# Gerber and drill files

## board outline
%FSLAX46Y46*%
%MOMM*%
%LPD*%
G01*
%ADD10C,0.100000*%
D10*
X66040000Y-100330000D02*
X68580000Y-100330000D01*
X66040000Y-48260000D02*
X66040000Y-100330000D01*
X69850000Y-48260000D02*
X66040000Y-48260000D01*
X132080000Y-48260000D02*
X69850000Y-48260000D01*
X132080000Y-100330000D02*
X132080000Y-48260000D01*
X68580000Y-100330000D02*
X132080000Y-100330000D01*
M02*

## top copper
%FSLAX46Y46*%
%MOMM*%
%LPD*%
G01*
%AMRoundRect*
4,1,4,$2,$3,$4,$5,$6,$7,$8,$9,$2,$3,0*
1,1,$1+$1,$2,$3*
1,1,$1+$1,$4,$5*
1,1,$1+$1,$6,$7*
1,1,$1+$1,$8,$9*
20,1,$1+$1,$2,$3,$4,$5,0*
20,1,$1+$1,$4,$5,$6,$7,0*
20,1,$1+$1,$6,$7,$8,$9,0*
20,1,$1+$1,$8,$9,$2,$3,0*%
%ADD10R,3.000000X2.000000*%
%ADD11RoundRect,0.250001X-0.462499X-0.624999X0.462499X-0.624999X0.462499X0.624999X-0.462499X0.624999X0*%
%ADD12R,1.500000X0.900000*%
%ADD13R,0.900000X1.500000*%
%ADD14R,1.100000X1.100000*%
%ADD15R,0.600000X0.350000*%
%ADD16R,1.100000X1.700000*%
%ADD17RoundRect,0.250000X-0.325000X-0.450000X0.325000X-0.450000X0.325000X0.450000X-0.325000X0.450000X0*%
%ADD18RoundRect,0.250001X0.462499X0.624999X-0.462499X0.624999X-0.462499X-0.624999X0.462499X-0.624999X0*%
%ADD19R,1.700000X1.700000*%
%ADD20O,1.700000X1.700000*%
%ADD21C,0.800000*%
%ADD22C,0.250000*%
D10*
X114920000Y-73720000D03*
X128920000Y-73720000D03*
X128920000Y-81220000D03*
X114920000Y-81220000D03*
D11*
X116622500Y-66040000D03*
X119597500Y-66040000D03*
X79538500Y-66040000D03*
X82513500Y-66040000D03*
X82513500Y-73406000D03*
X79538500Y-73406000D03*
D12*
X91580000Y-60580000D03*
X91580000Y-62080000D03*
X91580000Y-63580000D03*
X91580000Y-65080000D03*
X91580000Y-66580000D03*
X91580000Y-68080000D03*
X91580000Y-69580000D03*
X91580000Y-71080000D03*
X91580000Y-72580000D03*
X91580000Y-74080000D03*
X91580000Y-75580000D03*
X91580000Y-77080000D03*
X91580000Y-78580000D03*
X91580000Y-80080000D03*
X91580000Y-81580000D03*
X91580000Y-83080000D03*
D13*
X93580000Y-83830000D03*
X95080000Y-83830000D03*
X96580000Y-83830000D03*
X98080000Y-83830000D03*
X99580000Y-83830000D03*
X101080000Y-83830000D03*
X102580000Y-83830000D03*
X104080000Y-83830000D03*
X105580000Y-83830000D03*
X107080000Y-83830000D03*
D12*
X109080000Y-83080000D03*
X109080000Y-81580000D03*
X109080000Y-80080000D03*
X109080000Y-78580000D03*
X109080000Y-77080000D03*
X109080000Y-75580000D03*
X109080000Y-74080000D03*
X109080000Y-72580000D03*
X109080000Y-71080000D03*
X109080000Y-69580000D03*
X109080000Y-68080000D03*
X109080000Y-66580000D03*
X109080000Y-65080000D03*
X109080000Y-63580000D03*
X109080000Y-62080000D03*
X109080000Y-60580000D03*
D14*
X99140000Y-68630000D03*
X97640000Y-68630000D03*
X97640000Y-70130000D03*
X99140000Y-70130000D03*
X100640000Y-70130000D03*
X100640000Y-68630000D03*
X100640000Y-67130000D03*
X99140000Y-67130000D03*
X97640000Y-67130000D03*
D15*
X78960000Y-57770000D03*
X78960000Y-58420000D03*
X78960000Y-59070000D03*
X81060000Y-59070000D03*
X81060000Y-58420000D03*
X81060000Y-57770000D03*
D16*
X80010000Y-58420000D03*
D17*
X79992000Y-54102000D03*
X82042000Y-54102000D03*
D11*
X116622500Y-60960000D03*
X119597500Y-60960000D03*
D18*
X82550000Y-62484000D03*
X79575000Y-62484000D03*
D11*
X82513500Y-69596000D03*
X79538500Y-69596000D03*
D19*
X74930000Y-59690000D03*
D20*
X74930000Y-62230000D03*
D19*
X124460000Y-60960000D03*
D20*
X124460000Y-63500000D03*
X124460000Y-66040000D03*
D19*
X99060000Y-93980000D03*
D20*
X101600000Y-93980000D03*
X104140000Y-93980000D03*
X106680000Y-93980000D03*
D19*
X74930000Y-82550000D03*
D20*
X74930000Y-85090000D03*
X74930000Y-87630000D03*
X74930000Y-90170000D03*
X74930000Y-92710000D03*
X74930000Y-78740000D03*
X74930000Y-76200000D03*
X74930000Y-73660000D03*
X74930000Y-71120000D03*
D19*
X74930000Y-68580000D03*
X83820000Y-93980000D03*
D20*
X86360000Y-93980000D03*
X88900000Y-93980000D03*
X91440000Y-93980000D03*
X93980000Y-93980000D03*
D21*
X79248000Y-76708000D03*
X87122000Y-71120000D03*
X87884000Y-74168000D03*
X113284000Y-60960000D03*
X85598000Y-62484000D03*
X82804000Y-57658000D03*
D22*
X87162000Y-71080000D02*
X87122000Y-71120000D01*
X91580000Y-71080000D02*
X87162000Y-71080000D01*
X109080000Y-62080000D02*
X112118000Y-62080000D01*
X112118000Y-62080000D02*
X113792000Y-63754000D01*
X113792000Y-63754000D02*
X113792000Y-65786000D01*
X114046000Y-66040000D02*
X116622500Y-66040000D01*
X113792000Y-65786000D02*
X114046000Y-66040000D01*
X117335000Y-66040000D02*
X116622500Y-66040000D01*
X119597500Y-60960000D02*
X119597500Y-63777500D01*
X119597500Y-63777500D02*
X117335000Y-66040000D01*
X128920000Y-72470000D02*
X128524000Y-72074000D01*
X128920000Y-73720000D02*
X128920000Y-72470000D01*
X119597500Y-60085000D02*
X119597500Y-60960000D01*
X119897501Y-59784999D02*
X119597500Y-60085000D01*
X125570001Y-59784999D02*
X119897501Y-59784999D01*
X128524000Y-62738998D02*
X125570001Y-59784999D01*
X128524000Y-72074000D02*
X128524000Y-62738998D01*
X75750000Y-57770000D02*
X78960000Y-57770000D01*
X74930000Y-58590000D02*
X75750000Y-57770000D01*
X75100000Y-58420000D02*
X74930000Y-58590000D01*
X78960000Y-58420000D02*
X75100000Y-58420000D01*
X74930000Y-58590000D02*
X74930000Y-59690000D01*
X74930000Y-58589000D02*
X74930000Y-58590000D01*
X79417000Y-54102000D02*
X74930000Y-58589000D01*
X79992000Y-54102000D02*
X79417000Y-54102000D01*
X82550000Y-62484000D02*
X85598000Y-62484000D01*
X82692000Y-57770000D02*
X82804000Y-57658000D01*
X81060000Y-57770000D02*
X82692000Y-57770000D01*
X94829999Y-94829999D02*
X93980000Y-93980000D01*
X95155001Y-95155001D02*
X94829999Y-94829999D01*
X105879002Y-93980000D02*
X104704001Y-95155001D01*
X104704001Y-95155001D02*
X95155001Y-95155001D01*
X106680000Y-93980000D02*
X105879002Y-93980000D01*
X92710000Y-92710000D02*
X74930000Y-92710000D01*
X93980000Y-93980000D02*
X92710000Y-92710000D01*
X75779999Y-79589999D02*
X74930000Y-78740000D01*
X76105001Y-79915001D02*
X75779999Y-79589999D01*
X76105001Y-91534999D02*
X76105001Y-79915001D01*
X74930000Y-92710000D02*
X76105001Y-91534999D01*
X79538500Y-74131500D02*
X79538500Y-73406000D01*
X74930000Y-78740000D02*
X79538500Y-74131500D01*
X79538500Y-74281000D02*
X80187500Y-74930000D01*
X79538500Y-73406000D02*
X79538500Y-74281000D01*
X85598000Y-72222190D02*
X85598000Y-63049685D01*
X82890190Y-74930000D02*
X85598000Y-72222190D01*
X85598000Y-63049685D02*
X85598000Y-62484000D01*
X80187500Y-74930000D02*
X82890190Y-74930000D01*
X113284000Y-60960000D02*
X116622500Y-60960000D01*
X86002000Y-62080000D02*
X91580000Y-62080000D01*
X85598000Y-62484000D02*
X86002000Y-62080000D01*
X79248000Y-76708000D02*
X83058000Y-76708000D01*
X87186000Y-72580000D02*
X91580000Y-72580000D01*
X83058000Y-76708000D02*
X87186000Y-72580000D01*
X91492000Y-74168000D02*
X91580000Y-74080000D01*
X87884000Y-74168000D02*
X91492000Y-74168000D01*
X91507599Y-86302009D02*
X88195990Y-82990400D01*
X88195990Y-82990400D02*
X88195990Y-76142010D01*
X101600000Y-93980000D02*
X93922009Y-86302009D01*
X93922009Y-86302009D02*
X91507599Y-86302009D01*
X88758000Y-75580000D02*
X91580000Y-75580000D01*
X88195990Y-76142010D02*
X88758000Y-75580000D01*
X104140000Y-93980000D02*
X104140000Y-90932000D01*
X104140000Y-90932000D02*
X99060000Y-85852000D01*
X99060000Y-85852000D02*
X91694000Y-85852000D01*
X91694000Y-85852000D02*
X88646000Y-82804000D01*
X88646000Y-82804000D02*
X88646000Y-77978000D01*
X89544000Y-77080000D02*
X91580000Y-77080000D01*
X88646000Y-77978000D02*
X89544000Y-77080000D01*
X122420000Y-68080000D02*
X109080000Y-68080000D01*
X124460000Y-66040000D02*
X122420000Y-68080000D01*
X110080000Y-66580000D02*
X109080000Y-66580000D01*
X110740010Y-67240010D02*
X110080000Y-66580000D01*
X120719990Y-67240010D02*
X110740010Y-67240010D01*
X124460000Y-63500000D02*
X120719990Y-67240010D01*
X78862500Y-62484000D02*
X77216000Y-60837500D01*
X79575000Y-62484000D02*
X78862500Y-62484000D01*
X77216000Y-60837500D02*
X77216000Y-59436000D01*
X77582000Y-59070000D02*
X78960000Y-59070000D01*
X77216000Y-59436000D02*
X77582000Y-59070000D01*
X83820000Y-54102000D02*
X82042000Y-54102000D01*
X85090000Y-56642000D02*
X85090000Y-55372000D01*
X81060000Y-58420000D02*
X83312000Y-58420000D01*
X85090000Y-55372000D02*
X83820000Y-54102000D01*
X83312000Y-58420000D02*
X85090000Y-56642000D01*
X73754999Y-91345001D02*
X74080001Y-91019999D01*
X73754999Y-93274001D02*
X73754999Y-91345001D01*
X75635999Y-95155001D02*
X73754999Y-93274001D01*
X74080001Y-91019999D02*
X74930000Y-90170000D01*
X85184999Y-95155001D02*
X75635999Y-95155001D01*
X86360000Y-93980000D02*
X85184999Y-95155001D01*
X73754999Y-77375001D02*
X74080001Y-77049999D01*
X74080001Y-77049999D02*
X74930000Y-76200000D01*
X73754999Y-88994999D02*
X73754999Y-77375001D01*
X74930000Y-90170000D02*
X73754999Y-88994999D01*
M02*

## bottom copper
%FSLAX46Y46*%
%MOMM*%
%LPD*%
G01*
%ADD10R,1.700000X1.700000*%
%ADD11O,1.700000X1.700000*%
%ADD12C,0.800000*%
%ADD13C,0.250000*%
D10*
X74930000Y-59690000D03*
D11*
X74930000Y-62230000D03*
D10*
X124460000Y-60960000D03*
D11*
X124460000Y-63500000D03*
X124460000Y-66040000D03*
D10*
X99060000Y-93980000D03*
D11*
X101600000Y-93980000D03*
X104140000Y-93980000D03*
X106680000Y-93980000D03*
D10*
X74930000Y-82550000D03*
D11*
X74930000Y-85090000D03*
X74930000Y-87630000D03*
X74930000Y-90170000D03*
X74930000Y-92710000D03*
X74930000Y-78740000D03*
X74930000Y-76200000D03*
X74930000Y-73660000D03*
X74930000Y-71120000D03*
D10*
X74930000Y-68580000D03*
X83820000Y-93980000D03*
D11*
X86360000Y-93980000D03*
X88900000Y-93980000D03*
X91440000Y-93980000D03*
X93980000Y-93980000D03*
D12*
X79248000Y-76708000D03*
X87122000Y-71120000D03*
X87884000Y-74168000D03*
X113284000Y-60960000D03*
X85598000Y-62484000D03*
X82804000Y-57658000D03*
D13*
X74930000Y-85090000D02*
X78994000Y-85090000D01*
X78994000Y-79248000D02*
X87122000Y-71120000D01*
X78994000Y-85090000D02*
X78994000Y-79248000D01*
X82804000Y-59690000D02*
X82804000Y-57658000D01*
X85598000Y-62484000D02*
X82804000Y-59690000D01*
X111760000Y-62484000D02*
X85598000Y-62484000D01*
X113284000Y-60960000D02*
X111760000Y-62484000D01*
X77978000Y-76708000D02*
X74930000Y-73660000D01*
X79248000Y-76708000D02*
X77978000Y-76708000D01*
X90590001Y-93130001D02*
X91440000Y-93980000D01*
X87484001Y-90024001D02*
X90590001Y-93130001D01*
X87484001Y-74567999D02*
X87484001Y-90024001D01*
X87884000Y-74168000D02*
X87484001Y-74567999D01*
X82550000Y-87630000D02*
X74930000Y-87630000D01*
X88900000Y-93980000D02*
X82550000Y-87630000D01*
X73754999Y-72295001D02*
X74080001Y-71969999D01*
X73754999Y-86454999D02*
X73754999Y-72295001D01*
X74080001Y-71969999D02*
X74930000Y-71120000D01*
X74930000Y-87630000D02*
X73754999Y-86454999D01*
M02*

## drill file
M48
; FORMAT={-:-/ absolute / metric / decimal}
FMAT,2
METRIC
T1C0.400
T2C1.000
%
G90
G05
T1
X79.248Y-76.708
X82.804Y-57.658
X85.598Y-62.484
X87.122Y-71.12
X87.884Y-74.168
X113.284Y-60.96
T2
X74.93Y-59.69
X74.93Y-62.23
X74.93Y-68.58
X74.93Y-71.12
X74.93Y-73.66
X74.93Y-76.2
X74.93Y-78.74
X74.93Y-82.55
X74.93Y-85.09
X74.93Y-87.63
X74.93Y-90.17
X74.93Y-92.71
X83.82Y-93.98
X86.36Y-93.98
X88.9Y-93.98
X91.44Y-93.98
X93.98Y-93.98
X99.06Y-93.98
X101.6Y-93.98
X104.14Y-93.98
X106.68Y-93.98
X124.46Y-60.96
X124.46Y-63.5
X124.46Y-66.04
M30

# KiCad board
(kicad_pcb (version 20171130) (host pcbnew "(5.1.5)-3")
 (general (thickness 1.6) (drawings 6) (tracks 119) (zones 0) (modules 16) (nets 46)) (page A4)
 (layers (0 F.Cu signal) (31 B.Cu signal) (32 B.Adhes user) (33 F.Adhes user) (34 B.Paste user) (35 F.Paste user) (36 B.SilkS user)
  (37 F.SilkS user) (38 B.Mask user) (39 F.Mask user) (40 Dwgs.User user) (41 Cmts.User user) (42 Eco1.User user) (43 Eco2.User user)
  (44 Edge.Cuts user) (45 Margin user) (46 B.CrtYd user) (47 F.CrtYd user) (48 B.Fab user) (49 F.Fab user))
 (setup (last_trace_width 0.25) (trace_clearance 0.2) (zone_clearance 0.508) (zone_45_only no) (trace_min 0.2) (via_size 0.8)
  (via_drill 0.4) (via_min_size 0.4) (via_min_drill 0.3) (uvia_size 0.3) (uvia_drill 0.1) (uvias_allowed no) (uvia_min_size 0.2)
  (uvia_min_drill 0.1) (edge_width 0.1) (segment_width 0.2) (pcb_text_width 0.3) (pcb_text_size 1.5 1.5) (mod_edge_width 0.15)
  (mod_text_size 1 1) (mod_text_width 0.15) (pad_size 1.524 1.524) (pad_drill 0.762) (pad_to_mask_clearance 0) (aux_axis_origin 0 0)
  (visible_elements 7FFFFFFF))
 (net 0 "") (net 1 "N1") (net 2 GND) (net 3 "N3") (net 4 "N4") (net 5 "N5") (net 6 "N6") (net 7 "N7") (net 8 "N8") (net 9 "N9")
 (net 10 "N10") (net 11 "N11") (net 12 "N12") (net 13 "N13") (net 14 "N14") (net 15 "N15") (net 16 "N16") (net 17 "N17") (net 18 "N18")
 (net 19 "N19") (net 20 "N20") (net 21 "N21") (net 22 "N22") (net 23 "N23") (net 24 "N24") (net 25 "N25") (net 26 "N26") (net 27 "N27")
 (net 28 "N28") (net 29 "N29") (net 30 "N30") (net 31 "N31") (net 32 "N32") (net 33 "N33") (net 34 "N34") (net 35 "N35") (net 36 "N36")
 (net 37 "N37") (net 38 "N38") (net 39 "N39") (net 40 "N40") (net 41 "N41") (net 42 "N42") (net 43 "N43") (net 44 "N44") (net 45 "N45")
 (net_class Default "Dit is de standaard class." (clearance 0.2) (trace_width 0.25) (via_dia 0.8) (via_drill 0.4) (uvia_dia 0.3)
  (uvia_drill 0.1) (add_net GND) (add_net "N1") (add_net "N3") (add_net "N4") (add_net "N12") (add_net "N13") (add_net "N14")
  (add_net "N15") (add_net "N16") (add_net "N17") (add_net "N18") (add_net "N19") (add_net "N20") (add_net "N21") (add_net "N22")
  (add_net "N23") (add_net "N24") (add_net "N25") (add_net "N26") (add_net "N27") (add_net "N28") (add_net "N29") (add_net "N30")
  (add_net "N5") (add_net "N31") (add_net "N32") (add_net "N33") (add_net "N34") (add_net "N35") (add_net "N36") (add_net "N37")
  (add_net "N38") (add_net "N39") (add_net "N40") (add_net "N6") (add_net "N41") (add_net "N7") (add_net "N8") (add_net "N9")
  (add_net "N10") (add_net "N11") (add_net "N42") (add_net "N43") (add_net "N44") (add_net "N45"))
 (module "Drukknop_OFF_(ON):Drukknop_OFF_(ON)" (layer F.Cu) (at 121.92 77.47)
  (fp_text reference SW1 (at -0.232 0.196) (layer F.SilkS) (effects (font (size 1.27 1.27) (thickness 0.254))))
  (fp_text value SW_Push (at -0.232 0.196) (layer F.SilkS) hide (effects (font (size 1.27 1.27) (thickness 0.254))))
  (pad 4 smd rect (at -7 -3.75 90) (size 2 3) (layers F.Cu F.Paste F.Mask))
  (pad 3 smd rect (at 7 -3.75 90) (size 2 3) (layers F.Cu F.Paste F.Mask) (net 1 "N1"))
  (pad 2 smd rect (at 7 3.75 90) (size 2 3) (layers F.Cu F.Paste F.Mask))
  (pad 1 smd rect (at -7 3.75 90) (size 2 3) (layers F.Cu F.Paste F.Mask) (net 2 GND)))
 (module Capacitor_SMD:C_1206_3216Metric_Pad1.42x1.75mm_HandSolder (layer F.Cu) (at 118.11 66.04)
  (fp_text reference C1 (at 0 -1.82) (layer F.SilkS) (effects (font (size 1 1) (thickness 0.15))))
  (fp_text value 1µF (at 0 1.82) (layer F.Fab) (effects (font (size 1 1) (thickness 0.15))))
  (pad 1 smd roundrect (at -1.4875 0) (size 1.425 1.75) (layers F.Cu F.Paste F.Mask) (roundrect_rratio 0.175439) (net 1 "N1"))
  (pad 2 smd roundrect (at 1.4875 0) (size 1.425 1.75) (layers F.Cu F.Paste F.Mask) (roundrect_rratio 0.175439) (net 2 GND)))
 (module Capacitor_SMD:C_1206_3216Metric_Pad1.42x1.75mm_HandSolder (layer F.Cu) (at 81.026 66.04)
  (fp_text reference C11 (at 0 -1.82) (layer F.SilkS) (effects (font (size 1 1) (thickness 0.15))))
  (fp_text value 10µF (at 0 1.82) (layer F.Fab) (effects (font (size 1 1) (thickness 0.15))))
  (pad 1 smd roundrect (at -1.4875 0) (size 1.425 1.75) (layers F.Cu F.Paste F.Mask) (roundrect_rratio 0.175439) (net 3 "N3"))
  (pad 2 smd roundrect (at 1.4875 0) (size 1.425 1.75) (layers F.Cu F.Paste F.Mask) (roundrect_rratio 0.175439) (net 2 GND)))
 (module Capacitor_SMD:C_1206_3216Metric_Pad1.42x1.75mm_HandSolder (layer F.Cu) (at 81.026 73.406)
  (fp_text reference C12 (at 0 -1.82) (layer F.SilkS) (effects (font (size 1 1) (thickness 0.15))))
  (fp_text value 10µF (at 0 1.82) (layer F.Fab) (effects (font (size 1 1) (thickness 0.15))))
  (pad 2 smd roundrect (at 1.4875 0) (size 1.425 1.75) (layers F.Cu F.Paste F.Mask) (roundrect_rratio 0.175439) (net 2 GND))
  (pad 1 smd roundrect (at -1.4875 0) (size 1.425 1.75) (layers F.Cu F.Paste F.Mask) (roundrect_rratio 0.175439) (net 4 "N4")))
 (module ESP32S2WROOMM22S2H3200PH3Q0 (layer F.Cu) (at 100.33 68.58)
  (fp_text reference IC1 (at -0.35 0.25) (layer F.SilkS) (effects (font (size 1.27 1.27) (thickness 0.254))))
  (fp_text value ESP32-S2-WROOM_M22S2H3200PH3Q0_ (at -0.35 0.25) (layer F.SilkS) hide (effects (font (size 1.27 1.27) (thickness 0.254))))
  (pad 1 smd rect (at -8.75 -8 90) (size 0.9 1.5) (layers F.Cu F.Paste F.Mask) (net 2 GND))
  (pad 2 smd rect (at -8.75 -6.5 90) (size 0.9 1.5) (layers F.Cu F.Paste F.Mask) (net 4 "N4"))
  (pad 3 smd rect (at -8.75 -5 90) (size 0.9 1.5) (layers F.Cu F.Paste F.Mask) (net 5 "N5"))
  (pad 4 smd rect (at -8.75 -3.5 90) (size 0.9 1.5) (layers F.Cu F.Paste F.Mask) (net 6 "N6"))
  (pad 5 smd rect (at -8.75 -2 90) (size 0.9 1.5) (layers F.Cu F.Paste F.Mask) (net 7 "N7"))
  (pad 6 smd rect (at -8.75 -0.5 90) (size 0.9 1.5) (layers F.Cu F.Paste F.Mask) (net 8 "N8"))
  (pad 7 smd rect (at -8.75 1 90) (size 0.9 1.5) (layers F.Cu F.Paste F.Mask) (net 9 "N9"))
  (pad 8 smd rect (at -8.75 2.5 90) (size 0.9 1.5) (layers F.Cu F.Paste F.Mask) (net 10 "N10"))
  (pad 9 smd rect (at -8.75 4 90) (size 0.9 1.5) (layers F.Cu F.Paste F.Mask) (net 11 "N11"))
  (pad 10 smd rect (at -8.75 5.5 90) (size 0.9 1.5) (layers F.Cu F.Paste F.Mask) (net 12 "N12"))
  (pad 11 smd rect (at -8.75 7 90) (size 0.9 1.5) (layers F.Cu F.Paste F.Mask) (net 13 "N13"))
  (pad 12 smd rect (at -8.75 8.5 90) (size 0.9 1.5) (layers F.Cu F.Paste F.Mask) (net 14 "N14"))
  (pad 13 smd rect (at -8.75 10 90) (size 0.9 1.5) (layers F.Cu F.Paste F.Mask) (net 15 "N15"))
  (pad 14 smd rect (at -8.75 11.5 90) (size 0.9 1.5) (layers F.Cu F.Paste F.Mask) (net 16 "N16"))
  (pad 15 smd rect (at -8.75 13 90) (size 0.9 1.5) (layers F.Cu F.Paste F.Mask) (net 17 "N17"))
  (pad 16 smd rect (at -8.75 14.5 90) (size 0.9 1.5) (layers F.Cu F.Paste F.Mask) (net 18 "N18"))
  (pad 17 smd rect (at -6.75 15.25) (size 0.9 1.5) (layers F.Cu F.Paste F.Mask) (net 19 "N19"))
  (pad 18 smd rect (at -5.25 15.25) (size 0.9 1.5) (layers F.Cu F.Paste F.Mask) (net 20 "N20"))
  (pad 19 smd rect (at -3.75 15.25) (size 0.9 1.5) (layers F.Cu F.Paste F.Mask) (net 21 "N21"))
  (pad 20 smd rect (at -2.25 15.25) (size 0.9 1.5) (layers F.Cu F.Paste F.Mask) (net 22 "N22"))
  (pad 21 smd rect (at -0.75 15.25) (size 0.9 1.5) (layers F.Cu F.Paste F.Mask) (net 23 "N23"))
  (pad 22 smd rect (at 0.75 15.25) (size 0.9 1.5) (layers F.Cu F.Paste F.Mask) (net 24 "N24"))
  (pad 23 smd rect (at 2.25 15.25) (size 0.9 1.5) (layers F.Cu F.Paste F.Mask) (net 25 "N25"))
  (pad 24 smd rect (at 3.75 15.25) (size 0.9 1.5) (layers F.Cu F.Paste F.Mask) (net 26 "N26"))
  (pad 25 smd rect (at 5.25 15.25) (size 0.9 1.5) (layers F.Cu F.Paste F.Mask) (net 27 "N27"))
  (pad 26 smd rect (at 6.75 15.25) (size 0.9 1.5) (layers F.Cu F.Paste F.Mask) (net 2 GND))
  (pad 27 smd rect (at 8.75 14.5 90) (size 0.9 1.5) (layers F.Cu F.Paste F.Mask) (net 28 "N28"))
  (pad 28 smd rect (at 8.75 13 90) (size 0.9 1.5) (layers F.Cu F.Paste F.Mask) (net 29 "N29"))
  (pad 29 smd rect (at 8.75 11.5 90) (size 0.9 1.5) (layers F.Cu F.Paste F.Mask) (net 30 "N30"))
  (pad 30 smd rect (at 8.75 10 90) (size 0.9 1.5) (layers F.Cu F.Paste F.Mask) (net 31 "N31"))
  (pad 31 smd rect (at 8.75 8.5 90) (size 0.9 1.5) (layers F.Cu F.Paste F.Mask) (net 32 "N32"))
  (pad 32 smd rect (at 8.75 7 90) (size 0.9 1.5) (layers F.Cu F.Paste F.Mask) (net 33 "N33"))
  (pad 33 smd rect (at 8.75 5.5 90) (size 0.9 1.5) (layers F.Cu F.Paste F.Mask) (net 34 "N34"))
  (pad 34 smd rect (at 8.75 4 90) (size 0.9 1.5) (layers F.Cu F.Paste F.Mask) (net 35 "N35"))
  (pad 35 smd rect (at 8.75 2.5 90) (size 0.9 1.5) (layers F.Cu F.Paste F.Mask) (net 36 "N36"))
  (pad 36 smd rect (at 8.75 1 90) (size 0.9 1.5) (layers F.Cu F.Paste F.Mask) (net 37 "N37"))
  (pad 37 smd rect (at 8.75 -0.5 90) (size 0.9 1.5) (layers F.Cu F.Paste F.Mask) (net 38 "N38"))
  (pad 38 smd rect (at 8.75 -2 90) (size 0.9 1.5) (layers F.Cu F.Paste F.Mask) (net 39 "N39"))
  (pad 39 smd rect (at 8.75 -3.5 90) (size 0.9 1.5) (layers F.Cu F.Paste F.Mask) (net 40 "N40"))
  (pad 40 smd rect (at 8.75 -5 90) (size 0.9 1.5) (layers F.Cu F.Paste F.Mask) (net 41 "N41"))
  (pad 41 smd rect (at 8.75 -6.5 90) (size 0.9 1.5) (layers F.Cu F.Paste F.Mask) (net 1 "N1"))
  (pad 42 smd rect (at 8.75 -8 90) (size 0.9 1.5) (layers F.Cu F.Paste F.Mask) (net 2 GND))
  (pad 43 smd rect (at -1.19 0.05) (size 1.1 1.1) (layers F.Cu F.Paste F.Mask) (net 2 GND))
  (pad 44 smd rect (at -2.69 0.05) (size 1.1 1.1) (layers F.Cu F.Paste F.Mask) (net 2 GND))
  (pad 45 smd rect (at -2.69 1.55) (size 1.1 1.1) (layers F.Cu F.Paste F.Mask) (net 2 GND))
  (pad 46 smd rect (at -1.19 1.55) (size 1.1 1.1) (layers F.Cu F.Paste F.Mask) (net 2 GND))
  (pad 47 smd rect (at 0.31 1.55) (size 1.1 1.1) (layers F.Cu F.Paste F.Mask) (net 2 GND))
  (pad 48 smd rect (at 0.31 0.05) (size 1.1 1.1) (layers F.Cu F.Paste F.Mask) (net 2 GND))
  (pad 49 smd rect (at 0.31 -1.45) (size 1.1 1.1) (layers F.Cu F.Paste F.Mask) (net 2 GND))
  (pad 50 smd rect (at -1.19 -1.45) (size 1.1 1.1) (layers F.Cu F.Paste F.Mask) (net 2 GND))
  (pad 51 smd rect (at -2.69 -1.45) (size 1.1 1.1) (layers F.Cu F.Paste F.Mask) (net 2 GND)))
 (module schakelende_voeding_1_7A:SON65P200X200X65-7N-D (layer F.Cu) (at 80.01 58.42)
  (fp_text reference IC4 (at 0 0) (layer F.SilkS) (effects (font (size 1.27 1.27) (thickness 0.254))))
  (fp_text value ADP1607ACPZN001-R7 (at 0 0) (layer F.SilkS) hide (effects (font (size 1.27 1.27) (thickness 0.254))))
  (pad 1 smd rect (at -1.05 -0.65 90) (size 0.35 0.6) (layers F.Cu F.Paste F.Mask) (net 3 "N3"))
  (pad 2 smd rect (at -1.05 0 90) (size 0.35 0.6) (layers F.Cu F.Paste F.Mask) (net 3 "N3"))
  (pad 3 smd rect (at -1.05 0.65 90) (size 0.35 0.6) (layers F.Cu F.Paste F.Mask) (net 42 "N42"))
  (pad 4 smd rect (at 1.05 0.65 90) (size 0.35 0.6) (layers F.Cu F.Paste F.Mask) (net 2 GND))
  (pad 5 smd rect (at 1.05 0 90) (size 0.35 0.6) (layers F.Cu F.Paste F.Mask) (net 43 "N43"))
  (pad 6 smd rect (at 1.05 -0.65 90) (size 0.35 0.6) (layers F.Cu F.Paste F.Mask) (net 4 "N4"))
  (pad 7 smd rect (at 0 0) (size 1.1 1.7) (layers F.Cu F.Paste F.Mask) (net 2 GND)))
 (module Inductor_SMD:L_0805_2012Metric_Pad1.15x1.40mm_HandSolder (layer F.Cu) (at 81.017 54.102)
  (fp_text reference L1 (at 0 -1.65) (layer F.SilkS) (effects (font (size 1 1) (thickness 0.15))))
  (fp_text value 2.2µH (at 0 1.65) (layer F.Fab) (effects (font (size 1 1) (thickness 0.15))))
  (pad 1 smd roundrect (at -1.025 0) (size 1.15 1.4) (layers F.Cu F.Paste F.Mask) (roundrect_rratio 0.217391) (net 3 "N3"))
  (pad 2 smd roundrect (at 1.025 0) (size 1.15 1.4) (layers F.Cu F.Paste F.Mask) (roundrect_rratio 0.217391) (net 43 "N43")))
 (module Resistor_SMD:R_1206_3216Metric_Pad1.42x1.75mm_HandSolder (layer F.Cu) (at 118.11 60.96)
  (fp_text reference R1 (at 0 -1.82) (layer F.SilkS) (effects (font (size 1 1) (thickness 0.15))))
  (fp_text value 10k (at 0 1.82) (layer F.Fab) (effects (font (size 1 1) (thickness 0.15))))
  (pad 1 smd roundrect (at -1.4875 0) (size 1.425 1.75) (layers F.Cu F.Paste F.Mask) (roundrect_rratio 0.175439) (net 4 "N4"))
  (pad 2 smd roundrect (at 1.4875 0) (size 1.425 1.75) (layers F.Cu F.Paste F.Mask) (roundrect_rratio 0.175439) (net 1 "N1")))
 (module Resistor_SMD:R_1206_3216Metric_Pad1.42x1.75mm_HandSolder (layer F.Cu) (at 81.0625 62.484 180)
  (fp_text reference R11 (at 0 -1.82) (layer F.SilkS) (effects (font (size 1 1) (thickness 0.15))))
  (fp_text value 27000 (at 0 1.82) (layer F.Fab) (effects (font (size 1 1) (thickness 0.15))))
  (pad 1 smd roundrect (at -1.4875 0 180) (size 1.425 1.75) (layers F.Cu F.Paste F.Mask) (roundrect_rratio 0.175439) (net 4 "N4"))
  (pad 2 smd roundrect (at 1.4875 0 180) (size 1.425 1.75) (layers F.Cu F.Paste F.Mask) (roundrect_rratio 0.175439) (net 42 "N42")))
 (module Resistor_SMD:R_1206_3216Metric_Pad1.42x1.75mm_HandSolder (layer F.Cu) (at 81.026 69.596)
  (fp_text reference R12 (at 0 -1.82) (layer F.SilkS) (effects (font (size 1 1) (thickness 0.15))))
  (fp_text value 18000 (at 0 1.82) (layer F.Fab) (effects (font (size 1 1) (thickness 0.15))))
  (pad 2 smd roundrect (at 1.4875 0) (size 1.425 1.75) (layers F.Cu F.Paste F.Mask) (roundrect_rratio 0.175439) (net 2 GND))
  (pad 1 smd roundrect (at -1.4875 0) (size 1.425 1.75) (layers F.Cu F.Paste F.Mask) (roundrect_rratio 0.175439) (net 42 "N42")))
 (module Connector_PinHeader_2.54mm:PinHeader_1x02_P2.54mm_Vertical (layer F.Cu) (at 74.93 59.69)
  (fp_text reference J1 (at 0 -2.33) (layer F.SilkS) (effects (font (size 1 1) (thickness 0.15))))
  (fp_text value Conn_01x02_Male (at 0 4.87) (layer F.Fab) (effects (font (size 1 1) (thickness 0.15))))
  (pad 1 thru_hole rect (at 0 0) (size 1.7 1.7) (drill 1) (layers *.Cu *.Mask) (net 3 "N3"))
  (pad 2 thru_hole oval (at 0 2.54) (size 1.7 1.7) (drill 1) (layers *.Cu *.Mask) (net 2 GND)))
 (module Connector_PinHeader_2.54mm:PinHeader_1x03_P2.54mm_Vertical (layer F.Cu) (at 124.46 60.96)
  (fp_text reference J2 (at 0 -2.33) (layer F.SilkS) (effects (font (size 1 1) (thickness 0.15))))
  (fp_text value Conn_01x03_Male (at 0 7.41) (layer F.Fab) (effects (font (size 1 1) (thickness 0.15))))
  (pad 1 thru_hole rect (at 0 0) (size 1.7 1.7) (drill 1) (layers *.Cu *.Mask) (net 2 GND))
  (pad 2 thru_hole oval (at 0 2.54) (size 1.7 1.7) (drill 1) (layers *.Cu *.Mask) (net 39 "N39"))
  (pad 3 thru_hole oval (at 0 5.08) (size 1.7 1.7) (drill 1) (layers *.Cu *.Mask) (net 38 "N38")))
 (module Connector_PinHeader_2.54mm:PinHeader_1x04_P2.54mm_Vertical (layer F.Cu) (at 99.06 93.98 90)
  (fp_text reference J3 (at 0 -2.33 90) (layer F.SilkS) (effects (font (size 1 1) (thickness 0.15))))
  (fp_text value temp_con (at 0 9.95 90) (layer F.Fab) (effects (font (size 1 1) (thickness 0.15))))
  (pad 1 thru_hole rect (at 0 0 90) (size 1.7 1.7) (drill 1) (layers *.Cu *.Mask) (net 2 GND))
  (pad 2 thru_hole oval (at 0 2.54 90) (size 1.7 1.7) (drill 1) (layers *.Cu *.Mask) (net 13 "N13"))
  (pad 3 thru_hole oval (at 0 5.08 90) (size 1.7 1.7) (drill 1) (layers *.Cu *.Mask) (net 14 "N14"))
  (pad 4 thru_hole oval (at 0 7.62 90) (size 1.7 1.7) (drill 1) (layers *.Cu *.Mask) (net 4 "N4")))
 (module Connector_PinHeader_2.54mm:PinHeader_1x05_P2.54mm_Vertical (layer F.Cu) (at 74.93 82.55)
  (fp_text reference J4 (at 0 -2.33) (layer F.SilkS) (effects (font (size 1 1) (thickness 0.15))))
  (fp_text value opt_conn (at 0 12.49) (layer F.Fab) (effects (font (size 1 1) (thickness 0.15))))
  (pad 1 thru_hole rect (at 0 0) (size 1.7 1.7) (drill 1) (layers *.Cu *.Mask) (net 2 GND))
  (pad 2 thru_hole oval (at 0 2.54) (size 1.7 1.7) (drill 1) (layers *.Cu *.Mask) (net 10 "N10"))
  (pad 3 thru_hole oval (at 0 5.08) (size 1.7 1.7) (drill 1) (layers *.Cu *.Mask) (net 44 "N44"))
  (pad 4 thru_hole oval (at 0 7.62) (size 1.7 1.7) (drill 1) (layers *.Cu *.Mask) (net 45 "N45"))
  (pad 5 thru_hole oval (at 0 10.16) (size 1.7 1.7) (drill 1) (layers *.Cu *.Mask) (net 4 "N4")))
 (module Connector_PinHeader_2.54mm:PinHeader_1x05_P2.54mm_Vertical (layer F.Cu) (at 74.93 68.58)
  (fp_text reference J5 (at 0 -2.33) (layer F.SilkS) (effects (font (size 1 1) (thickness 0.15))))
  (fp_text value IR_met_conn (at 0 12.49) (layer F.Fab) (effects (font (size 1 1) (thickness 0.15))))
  (pad 5 thru_hole oval (at 0 10.16) (size 1.7 1.7) (drill 1) (layers *.Cu *.Mask) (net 4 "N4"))
  (pad 4 thru_hole oval (at 0 7.62) (size 1.7 1.7) (drill 1) (layers *.Cu *.Mask) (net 45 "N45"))
  (pad 3 thru_hole oval (at 0 5.08) (size 1.7 1.7) (drill 1) (layers *.Cu *.Mask) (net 11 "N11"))
  (pad 2 thru_hole oval (at 0 2.54) (size 1.7 1.7) (drill 1) (layers *.Cu *.Mask) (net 44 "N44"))
  (pad 1 thru_hole rect (at 0 0) (size 1.7 1.7) (drill 1) (layers *.Cu *.Mask) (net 2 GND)))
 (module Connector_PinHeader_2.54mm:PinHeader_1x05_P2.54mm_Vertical (layer F.Cu) (at 83.82 93.98 90)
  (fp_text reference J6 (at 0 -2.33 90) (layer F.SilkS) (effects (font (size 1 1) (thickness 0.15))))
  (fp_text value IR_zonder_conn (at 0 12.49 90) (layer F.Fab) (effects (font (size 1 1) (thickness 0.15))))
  (pad 1 thru_hole rect (at 0 0 90) (size 1.7 1.7) (drill 1) (layers *.Cu *.Mask) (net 2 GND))
  (pad 2 thru_hole oval (at 0 2.54 90) (size 1.7 1.7) (drill 1) (layers *.Cu *.Mask) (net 45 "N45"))
  (pad 3 thru_hole oval (at 0 5.08 90) (size 1.7 1.7) (drill 1) (layers *.Cu *.Mask) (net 44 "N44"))
  (pad 4 thru_hole oval (at 0 7.62 90) (size 1.7 1.7) (drill 1) (layers *.Cu *.Mask) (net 12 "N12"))
  (pad 5 thru_hole oval (at 0 10.16 90) (size 1.7 1.7) (drill 1) (layers *.Cu *.Mask) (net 4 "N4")))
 (gr_line (start 66.04 100.33) (end 68.58 100.33) (layer Edge.Cuts) (width 0.1))
 (gr_line (start 66.04 48.26) (end 66.04 100.33) (layer Edge.Cuts) (width 0.1))
 (gr_line (start 69.85 48.26) (end 66.04 48.26) (layer Edge.Cuts) (width 0.1))
 (gr_line (start 132.08 48.26) (end 69.85 48.26) (layer Edge.Cuts) (width 0.1))
 (gr_line (start 132.08 100.33) (end 132.08 48.26) (layer Edge.Cuts) (width 0.1))
 (gr_line (start 68.58 100.33) (end 132.08 100.33) (layer Edge.Cuts) (width 0.1))
 (via (at 79.248 76.708) (size 0.8) (drill 0.4) (layers F.Cu B.Cu) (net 11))
 (via (at 87.122 71.12) (size 0.8) (drill 0.4) (layers F.Cu B.Cu) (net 10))
 (segment (start 87.162 71.08) (end 87.122 71.12) (width 0.25) (layer F.Cu) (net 10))
 (segment (start 91.58 71.08) (end 87.162 71.08) (width 0.25) (layer F.Cu) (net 10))
 (segment (start 74.93 85.09) (end 78.994 85.09) (width 0.25) (layer B.Cu) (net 10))
 (segment (start 78.994 79.248) (end 87.122 71.12) (width 0.25) (layer B.Cu) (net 10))
 (segment (start 78.994 85.09) (end 78.994 79.248) (width 0.25) (layer B.Cu) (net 10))
 (via (at 87.884 74.168) (size 0.8) (drill 0.4) (layers F.Cu B.Cu) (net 12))
 (via (at 113.284 60.96) (size 0.8) (drill 0.4) (layers F.Cu B.Cu) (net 4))
 (segment (start 109.08 62.08) (end 112.118 62.08) (width 0.25) (layer F.Cu) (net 1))
 (segment (start 112.118 62.08) (end 113.792 63.754) (width 0.25) (layer F.Cu) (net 1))
 (segment (start 113.792 63.754) (end 113.792 65.786) (width 0.25) (layer F.Cu) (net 1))
 (segment (start 114.046 66.04) (end 116.6225 66.04) (width 0.25) (layer F.Cu) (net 1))
 (segment (start 113.792 65.786) (end 114.046 66.04) (width 0.25) (layer F.Cu) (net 1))
 (segment (start 117.335 66.04) (end 116.6225 66.04) (width 0.25) (layer F.Cu) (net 1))
 (segment (start 119.5975 60.96) (end 119.5975 63.7775) (width 0.25) (layer F.Cu) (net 1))
 (segment (start 119.5975 63.7775) (end 117.335 66.04) (width 0.25) (layer F.Cu) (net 1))
 (segment (start 128.92 72.47) (end 128.524 72.074) (width 0.25) (layer F.Cu) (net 1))
 (segment (start 128.92 73.72) (end 128.92 72.47) (width 0.25) (layer F.Cu) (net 1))
 (segment (start 119.5975 60.085) (end 119.5975 60.96) (width 0.25) (layer F.Cu) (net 1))
 (segment (start 119.897501 59.784999) (end 119.5975 60.085) (width 0.25) (layer F.Cu) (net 1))
 (segment (start 125.570001 59.784999) (end 119.897501 59.784999) (width 0.25) (layer F.Cu) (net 1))
 (segment (start 128.524 62.738998) (end 125.570001 59.784999) (width 0.25) (layer F.Cu) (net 1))
 (segment (start 128.524 72.074) (end 128.524 62.738998) (width 0.25) (layer F.Cu) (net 1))
 (via (at 85.598 62.484) (size 0.8) (drill 0.4) (layers F.Cu B.Cu) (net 4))
 (via (at 82.804 57.658) (size 0.8) (drill 0.4) (layers F.Cu B.Cu) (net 4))
 (segment (start 75.75 57.77) (end 78.96 57.77) (width 0.25) (layer F.Cu) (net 3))
 (segment (start 74.93 58.59) (end 75.75 57.77) (width 0.25) (layer F.Cu) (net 3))
 (segment (start 75.1 58.42) (end 74.93 58.59) (width 0.25) (layer F.Cu) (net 3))
 (segment (start 78.96 58.42) (end 75.1 58.42) (width 0.25) (layer F.Cu) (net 3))
 (segment (start 74.93 58.59) (end 74.93 59.69) (width 0.25) (layer F.Cu) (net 3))
 (segment (start 74.93 58.589) (end 74.93 58.59) (width 0.25) (layer F.Cu) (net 3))
 (segment (start 79.417 54.102) (end 74.93 58.589) (width 0.25) (layer F.Cu) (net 3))
 (segment (start 79.992 54.102) (end 79.417 54.102) (width 0.25) (layer F.Cu) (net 3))
 (segment (start 82.55 62.484) (end 85.598 62.484) (width 0.25) (layer F.Cu) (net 4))
 (segment (start 82.692 57.77) (end 82.804 57.658) (width 0.25) (layer F.Cu) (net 4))
 (segment (start 81.06 57.77) (end 82.692 57.77) (width 0.25) (layer F.Cu) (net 4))
 (segment (start 82.804 59.69) (end 82.804 57.658) (width 0.25) (layer B.Cu) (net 4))
 (segment (start 85.598 62.484) (end 82.804 59.69) (width 0.25) (layer B.Cu) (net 4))
 (segment (start 94.829999 94.829999) (end 93.98 93.98) (width 0.25) (layer F.Cu) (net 4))
 (segment (start 95.155001 95.155001) (end 94.829999 94.829999) (width 0.25) (layer F.Cu) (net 4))
 (segment (start 105.879002 93.98) (end 104.704001 95.155001) (width 0.25) (layer F.Cu) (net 4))
 (segment (start 104.704001 95.155001) (end 95.155001 95.155001) (width 0.25) (layer F.Cu) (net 4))
 (segment (start 106.68 93.98) (end 105.879002 93.98) (width 0.25) (layer F.Cu) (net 4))
 (segment (start 92.71 92.71) (end 74.93 92.71) (width 0.25) (layer F.Cu) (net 4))
 (segment (start 93.98 93.98) (end 92.71 92.71) (width 0.25) (layer F.Cu) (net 4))
 (segment (start 75.779999 79.589999) (end 74.93 78.74) (width 0.25) (layer F.Cu) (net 4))
 (segment (start 76.105001 79.915001) (end 75.779999 79.589999) (width 0.25) (layer F.Cu) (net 4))
 (segment (start 76.105001 91.534999) (end 76.105001 79.915001) (width 0.25) (layer F.Cu) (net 4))
 (segment (start 74.93 92.71) (end 76.105001 91.534999) (width 0.25) (layer F.Cu) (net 4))
 (segment (start 79.5385 74.1315) (end 79.5385 73.406) (width 0.25) (layer F.Cu) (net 4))
 (segment (start 74.93 78.74) (end 79.5385 74.1315) (width 0.25) (layer F.Cu) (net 4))
 (segment (start 79.5385 74.281) (end 80.1875 74.93) (width 0.25) (layer F.Cu) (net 4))
 (segment (start 79.5385 73.406) (end 79.5385 74.281) (width 0.25) (layer F.Cu) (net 4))
 (segment (start 85.598 72.22219) (end 85.598 63.049685) (width 0.25) (layer F.Cu) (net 4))
 (segment (start 82.89019 74.93) (end 85.598 72.22219) (width 0.25) (layer F.Cu) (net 4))
 (segment (start 85.598 63.049685) (end 85.598 62.484) (width 0.25) (layer F.Cu) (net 4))
 (segment (start 80.1875 74.93) (end 82.89019 74.93) (width 0.25) (layer F.Cu) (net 4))
 (segment (start 113.284 60.96) (end 116.6225 60.96) (width 0.25) (layer F.Cu) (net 4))
 (segment (start 111.76 62.484) (end 85.598 62.484) (width 0.25) (layer B.Cu) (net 4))
 (segment (start 113.284 60.96) (end 111.76 62.484) (width 0.25) (layer B.Cu) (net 4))
 (segment (start 86.002 62.08) (end 91.58 62.08) (width 0.25) (layer F.Cu) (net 4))
 (segment (start 85.598 62.484) (end 86.002 62.08) (width 0.25) (layer F.Cu) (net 4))
 (segment (start 77.978 76.708) (end 74.93 73.66) (width 0.25) (layer B.Cu) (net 11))
 (segment (start 79.248 76.708) (end 77.978 76.708) (width 0.25) (layer B.Cu) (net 11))
 (segment (start 79.248 76.708) (end 83.058 76.708) (width 0.25) (layer F.Cu) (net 11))
 (segment (start 87.186 72.58) (end 91.58 72.58) (width 0.25) (layer F.Cu) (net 11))
 (segment (start 83.058 76.708) (end 87.186 72.58) (width 0.25) (layer F.Cu) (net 11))
 (segment (start 91.492 74.168) (end 91.58 74.08) (width 0.25) (layer F.Cu) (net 12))
 (segment (start 87.884 74.168) (end 91.492 74.168) (width 0.25) (layer F.Cu) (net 12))
 (segment (start 90.590001 93.130001) (end 91.44 93.98) (width 0.25) (layer B.Cu) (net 12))
 (segment (start 87.484001 90.024001) (end 90.590001 93.130001) (width 0.25) (layer B.Cu) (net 12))
 (segment (start 87.484001 74.567999) (end 87.484001 90.024001) (width 0.25) (layer B.Cu) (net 12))
 (segment (start 87.884 74.168) (end 87.484001 74.567999) (width 0.25) (layer B.Cu) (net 12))
 (segment (start 91.507599 86.302009) (end 88.19599 82.9904) (width 0.25) (layer F.Cu) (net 13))
 (segment (start 88.19599 82.9904) (end 88.19599 76.14201) (width 0.25) (layer F.Cu) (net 13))
 (segment (start 101.6 93.98) (end 93.922009 86.302009) (width 0.25) (layer F.Cu) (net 13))
 (segment (start 93.922009 86.302009) (end 91.507599 86.302009) (width 0.25) (layer F.Cu) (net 13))
 (segment (start 88.758 75.58) (end 91.58 75.58) (width 0.25) (layer F.Cu) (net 13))
 (segment (start 88.19599 76.14201) (end 88.758 75.58) (width 0.25) (layer F.Cu) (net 13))
 (segment (start 104.14 93.98) (end 104.14 90.932) (width 0.25) (layer F.Cu) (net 14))
 (segment (start 104.14 90.932) (end 99.06 85.852) (width 0.25) (layer F.Cu) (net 14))
 (segment (start 99.06 85.852) (end 91.694 85.852) (width 0.25) (layer F.Cu) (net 14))
 (segment (start 91.694 85.852) (end 88.646 82.804) (width 0.25) (layer F.Cu) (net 14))
 (segment (start 88.646 82.804) (end 88.646 77.978) (width 0.25) (layer F.Cu) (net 14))
 (segment (start 89.544 77.08) (end 91.58 77.08) (width 0.25) (layer F.Cu) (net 14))
 (segment (start 88.646 77.978) (end 89.544 77.08) (width 0.25) (layer F.Cu) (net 14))
 (segment (start 122.42 68.08) (end 109.08 68.08) (width 0.25) (layer F.Cu) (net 38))
 (segment (start 124.46 66.04) (end 122.42 68.08) (width 0.25) (layer F.Cu) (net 38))
 (segment (start 110.08 66.58) (end 109.08 66.58) (width 0.25) (layer F.Cu) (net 39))
 (segment (start 110.74001 67.24001) (end 110.08 66.58) (width 0.25) (layer F.Cu) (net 39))
 (segment (start 120.71999 67.24001) (end 110.74001 67.24001) (width 0.25) (layer F.Cu) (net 39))
 (segment (start 124.46 63.5) (end 120.71999 67.24001) (width 0.25) (layer F.Cu) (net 39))
 (segment (start 78.8625 62.484) (end 77.216 60.8375) (width 0.25) (layer F.Cu) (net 42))
 (segment (start 79.575 62.484) (end 78.8625 62.484) (width 0.25) (layer F.Cu) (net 42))
 (segment (start 77.216 60.8375) (end 77.216 59.436) (width 0.25) (layer F.Cu) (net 42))
 (segment (start 77.582 59.07) (end 78.96 59.07) (width 0.25) (layer F.Cu) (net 42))
 (segment (start 77.216 59.436) (end 77.582 59.07) (width 0.25) (layer F.Cu) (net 42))
 (segment (start 83.82 54.102) (end 82.042 54.102) (width 0.25) (layer F.Cu) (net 43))
 (segment (start 85.09 56.642) (end 85.09 55.372) (width 0.25) (layer F.Cu) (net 43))
 (segment (start 81.06 58.42) (end 83.312 58.42) (width 0.25) (layer F.Cu) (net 43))
 (segment (start 85.09 55.372) (end 83.82 54.102) (width 0.25) (layer F.Cu) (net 43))
 (segment (start 83.312 58.42) (end 85.09 56.642) (width 0.25) (layer F.Cu) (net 43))
 (segment (start 82.55 87.63) (end 74.93 87.63) (width 0.25) (layer B.Cu) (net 44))
 (segment (start 88.9 93.98) (end 82.55 87.63) (width 0.25) (layer B.Cu) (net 44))
 (segment (start 73.754999 72.295001) (end 74.080001 71.969999) (width 0.25) (layer B.Cu) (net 44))
 (segment (start 73.754999 86.454999) (end 73.754999 72.295001) (width 0.25) (layer B.Cu) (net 44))
 (segment (start 74.080001 71.969999) (end 74.93 71.12) (width 0.25) (layer B.Cu) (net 44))
 (segment (start 74.93 87.63) (end 73.754999 86.454999) (width 0.25) (layer B.Cu) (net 44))
 (segment (start 73.754999 91.345001) (end 74.080001 91.019999) (width 0.25) (layer F.Cu) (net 45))
 (segment (start 73.754999 93.274001) (end 73.754999 91.345001) (width 0.25) (layer F.Cu) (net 45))
 (segment (start 75.635999 95.155001) (end 73.754999 93.274001) (width 0.25) (layer F.Cu) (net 45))
 (segment (start 74.080001 91.019999) (end 74.93 90.17) (width 0.25) (layer F.Cu) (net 45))
 (segment (start 85.184999 95.155001) (end 75.635999 95.155001) (width 0.25) (layer F.Cu) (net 45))
 (segment (start 86.36 93.98) (end 85.184999 95.155001) (width 0.25) (layer F.Cu) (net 45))
 (segment (start 73.754999 77.375001) (end 74.080001 77.049999) (width 0.25) (layer F.Cu) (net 45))
 (segment (start 74.080001 77.049999) (end 74.93 76.2) (width 0.25) (layer F.Cu) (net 45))
 (segment (start 73.754999 88.994999) (end 73.754999 77.375001) (width 0.25) (layer F.Cu) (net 45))
 (segment (start 74.93 90.17) (end 73.754999 88.994999) (width 0.25) (layer F.Cu) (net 45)))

